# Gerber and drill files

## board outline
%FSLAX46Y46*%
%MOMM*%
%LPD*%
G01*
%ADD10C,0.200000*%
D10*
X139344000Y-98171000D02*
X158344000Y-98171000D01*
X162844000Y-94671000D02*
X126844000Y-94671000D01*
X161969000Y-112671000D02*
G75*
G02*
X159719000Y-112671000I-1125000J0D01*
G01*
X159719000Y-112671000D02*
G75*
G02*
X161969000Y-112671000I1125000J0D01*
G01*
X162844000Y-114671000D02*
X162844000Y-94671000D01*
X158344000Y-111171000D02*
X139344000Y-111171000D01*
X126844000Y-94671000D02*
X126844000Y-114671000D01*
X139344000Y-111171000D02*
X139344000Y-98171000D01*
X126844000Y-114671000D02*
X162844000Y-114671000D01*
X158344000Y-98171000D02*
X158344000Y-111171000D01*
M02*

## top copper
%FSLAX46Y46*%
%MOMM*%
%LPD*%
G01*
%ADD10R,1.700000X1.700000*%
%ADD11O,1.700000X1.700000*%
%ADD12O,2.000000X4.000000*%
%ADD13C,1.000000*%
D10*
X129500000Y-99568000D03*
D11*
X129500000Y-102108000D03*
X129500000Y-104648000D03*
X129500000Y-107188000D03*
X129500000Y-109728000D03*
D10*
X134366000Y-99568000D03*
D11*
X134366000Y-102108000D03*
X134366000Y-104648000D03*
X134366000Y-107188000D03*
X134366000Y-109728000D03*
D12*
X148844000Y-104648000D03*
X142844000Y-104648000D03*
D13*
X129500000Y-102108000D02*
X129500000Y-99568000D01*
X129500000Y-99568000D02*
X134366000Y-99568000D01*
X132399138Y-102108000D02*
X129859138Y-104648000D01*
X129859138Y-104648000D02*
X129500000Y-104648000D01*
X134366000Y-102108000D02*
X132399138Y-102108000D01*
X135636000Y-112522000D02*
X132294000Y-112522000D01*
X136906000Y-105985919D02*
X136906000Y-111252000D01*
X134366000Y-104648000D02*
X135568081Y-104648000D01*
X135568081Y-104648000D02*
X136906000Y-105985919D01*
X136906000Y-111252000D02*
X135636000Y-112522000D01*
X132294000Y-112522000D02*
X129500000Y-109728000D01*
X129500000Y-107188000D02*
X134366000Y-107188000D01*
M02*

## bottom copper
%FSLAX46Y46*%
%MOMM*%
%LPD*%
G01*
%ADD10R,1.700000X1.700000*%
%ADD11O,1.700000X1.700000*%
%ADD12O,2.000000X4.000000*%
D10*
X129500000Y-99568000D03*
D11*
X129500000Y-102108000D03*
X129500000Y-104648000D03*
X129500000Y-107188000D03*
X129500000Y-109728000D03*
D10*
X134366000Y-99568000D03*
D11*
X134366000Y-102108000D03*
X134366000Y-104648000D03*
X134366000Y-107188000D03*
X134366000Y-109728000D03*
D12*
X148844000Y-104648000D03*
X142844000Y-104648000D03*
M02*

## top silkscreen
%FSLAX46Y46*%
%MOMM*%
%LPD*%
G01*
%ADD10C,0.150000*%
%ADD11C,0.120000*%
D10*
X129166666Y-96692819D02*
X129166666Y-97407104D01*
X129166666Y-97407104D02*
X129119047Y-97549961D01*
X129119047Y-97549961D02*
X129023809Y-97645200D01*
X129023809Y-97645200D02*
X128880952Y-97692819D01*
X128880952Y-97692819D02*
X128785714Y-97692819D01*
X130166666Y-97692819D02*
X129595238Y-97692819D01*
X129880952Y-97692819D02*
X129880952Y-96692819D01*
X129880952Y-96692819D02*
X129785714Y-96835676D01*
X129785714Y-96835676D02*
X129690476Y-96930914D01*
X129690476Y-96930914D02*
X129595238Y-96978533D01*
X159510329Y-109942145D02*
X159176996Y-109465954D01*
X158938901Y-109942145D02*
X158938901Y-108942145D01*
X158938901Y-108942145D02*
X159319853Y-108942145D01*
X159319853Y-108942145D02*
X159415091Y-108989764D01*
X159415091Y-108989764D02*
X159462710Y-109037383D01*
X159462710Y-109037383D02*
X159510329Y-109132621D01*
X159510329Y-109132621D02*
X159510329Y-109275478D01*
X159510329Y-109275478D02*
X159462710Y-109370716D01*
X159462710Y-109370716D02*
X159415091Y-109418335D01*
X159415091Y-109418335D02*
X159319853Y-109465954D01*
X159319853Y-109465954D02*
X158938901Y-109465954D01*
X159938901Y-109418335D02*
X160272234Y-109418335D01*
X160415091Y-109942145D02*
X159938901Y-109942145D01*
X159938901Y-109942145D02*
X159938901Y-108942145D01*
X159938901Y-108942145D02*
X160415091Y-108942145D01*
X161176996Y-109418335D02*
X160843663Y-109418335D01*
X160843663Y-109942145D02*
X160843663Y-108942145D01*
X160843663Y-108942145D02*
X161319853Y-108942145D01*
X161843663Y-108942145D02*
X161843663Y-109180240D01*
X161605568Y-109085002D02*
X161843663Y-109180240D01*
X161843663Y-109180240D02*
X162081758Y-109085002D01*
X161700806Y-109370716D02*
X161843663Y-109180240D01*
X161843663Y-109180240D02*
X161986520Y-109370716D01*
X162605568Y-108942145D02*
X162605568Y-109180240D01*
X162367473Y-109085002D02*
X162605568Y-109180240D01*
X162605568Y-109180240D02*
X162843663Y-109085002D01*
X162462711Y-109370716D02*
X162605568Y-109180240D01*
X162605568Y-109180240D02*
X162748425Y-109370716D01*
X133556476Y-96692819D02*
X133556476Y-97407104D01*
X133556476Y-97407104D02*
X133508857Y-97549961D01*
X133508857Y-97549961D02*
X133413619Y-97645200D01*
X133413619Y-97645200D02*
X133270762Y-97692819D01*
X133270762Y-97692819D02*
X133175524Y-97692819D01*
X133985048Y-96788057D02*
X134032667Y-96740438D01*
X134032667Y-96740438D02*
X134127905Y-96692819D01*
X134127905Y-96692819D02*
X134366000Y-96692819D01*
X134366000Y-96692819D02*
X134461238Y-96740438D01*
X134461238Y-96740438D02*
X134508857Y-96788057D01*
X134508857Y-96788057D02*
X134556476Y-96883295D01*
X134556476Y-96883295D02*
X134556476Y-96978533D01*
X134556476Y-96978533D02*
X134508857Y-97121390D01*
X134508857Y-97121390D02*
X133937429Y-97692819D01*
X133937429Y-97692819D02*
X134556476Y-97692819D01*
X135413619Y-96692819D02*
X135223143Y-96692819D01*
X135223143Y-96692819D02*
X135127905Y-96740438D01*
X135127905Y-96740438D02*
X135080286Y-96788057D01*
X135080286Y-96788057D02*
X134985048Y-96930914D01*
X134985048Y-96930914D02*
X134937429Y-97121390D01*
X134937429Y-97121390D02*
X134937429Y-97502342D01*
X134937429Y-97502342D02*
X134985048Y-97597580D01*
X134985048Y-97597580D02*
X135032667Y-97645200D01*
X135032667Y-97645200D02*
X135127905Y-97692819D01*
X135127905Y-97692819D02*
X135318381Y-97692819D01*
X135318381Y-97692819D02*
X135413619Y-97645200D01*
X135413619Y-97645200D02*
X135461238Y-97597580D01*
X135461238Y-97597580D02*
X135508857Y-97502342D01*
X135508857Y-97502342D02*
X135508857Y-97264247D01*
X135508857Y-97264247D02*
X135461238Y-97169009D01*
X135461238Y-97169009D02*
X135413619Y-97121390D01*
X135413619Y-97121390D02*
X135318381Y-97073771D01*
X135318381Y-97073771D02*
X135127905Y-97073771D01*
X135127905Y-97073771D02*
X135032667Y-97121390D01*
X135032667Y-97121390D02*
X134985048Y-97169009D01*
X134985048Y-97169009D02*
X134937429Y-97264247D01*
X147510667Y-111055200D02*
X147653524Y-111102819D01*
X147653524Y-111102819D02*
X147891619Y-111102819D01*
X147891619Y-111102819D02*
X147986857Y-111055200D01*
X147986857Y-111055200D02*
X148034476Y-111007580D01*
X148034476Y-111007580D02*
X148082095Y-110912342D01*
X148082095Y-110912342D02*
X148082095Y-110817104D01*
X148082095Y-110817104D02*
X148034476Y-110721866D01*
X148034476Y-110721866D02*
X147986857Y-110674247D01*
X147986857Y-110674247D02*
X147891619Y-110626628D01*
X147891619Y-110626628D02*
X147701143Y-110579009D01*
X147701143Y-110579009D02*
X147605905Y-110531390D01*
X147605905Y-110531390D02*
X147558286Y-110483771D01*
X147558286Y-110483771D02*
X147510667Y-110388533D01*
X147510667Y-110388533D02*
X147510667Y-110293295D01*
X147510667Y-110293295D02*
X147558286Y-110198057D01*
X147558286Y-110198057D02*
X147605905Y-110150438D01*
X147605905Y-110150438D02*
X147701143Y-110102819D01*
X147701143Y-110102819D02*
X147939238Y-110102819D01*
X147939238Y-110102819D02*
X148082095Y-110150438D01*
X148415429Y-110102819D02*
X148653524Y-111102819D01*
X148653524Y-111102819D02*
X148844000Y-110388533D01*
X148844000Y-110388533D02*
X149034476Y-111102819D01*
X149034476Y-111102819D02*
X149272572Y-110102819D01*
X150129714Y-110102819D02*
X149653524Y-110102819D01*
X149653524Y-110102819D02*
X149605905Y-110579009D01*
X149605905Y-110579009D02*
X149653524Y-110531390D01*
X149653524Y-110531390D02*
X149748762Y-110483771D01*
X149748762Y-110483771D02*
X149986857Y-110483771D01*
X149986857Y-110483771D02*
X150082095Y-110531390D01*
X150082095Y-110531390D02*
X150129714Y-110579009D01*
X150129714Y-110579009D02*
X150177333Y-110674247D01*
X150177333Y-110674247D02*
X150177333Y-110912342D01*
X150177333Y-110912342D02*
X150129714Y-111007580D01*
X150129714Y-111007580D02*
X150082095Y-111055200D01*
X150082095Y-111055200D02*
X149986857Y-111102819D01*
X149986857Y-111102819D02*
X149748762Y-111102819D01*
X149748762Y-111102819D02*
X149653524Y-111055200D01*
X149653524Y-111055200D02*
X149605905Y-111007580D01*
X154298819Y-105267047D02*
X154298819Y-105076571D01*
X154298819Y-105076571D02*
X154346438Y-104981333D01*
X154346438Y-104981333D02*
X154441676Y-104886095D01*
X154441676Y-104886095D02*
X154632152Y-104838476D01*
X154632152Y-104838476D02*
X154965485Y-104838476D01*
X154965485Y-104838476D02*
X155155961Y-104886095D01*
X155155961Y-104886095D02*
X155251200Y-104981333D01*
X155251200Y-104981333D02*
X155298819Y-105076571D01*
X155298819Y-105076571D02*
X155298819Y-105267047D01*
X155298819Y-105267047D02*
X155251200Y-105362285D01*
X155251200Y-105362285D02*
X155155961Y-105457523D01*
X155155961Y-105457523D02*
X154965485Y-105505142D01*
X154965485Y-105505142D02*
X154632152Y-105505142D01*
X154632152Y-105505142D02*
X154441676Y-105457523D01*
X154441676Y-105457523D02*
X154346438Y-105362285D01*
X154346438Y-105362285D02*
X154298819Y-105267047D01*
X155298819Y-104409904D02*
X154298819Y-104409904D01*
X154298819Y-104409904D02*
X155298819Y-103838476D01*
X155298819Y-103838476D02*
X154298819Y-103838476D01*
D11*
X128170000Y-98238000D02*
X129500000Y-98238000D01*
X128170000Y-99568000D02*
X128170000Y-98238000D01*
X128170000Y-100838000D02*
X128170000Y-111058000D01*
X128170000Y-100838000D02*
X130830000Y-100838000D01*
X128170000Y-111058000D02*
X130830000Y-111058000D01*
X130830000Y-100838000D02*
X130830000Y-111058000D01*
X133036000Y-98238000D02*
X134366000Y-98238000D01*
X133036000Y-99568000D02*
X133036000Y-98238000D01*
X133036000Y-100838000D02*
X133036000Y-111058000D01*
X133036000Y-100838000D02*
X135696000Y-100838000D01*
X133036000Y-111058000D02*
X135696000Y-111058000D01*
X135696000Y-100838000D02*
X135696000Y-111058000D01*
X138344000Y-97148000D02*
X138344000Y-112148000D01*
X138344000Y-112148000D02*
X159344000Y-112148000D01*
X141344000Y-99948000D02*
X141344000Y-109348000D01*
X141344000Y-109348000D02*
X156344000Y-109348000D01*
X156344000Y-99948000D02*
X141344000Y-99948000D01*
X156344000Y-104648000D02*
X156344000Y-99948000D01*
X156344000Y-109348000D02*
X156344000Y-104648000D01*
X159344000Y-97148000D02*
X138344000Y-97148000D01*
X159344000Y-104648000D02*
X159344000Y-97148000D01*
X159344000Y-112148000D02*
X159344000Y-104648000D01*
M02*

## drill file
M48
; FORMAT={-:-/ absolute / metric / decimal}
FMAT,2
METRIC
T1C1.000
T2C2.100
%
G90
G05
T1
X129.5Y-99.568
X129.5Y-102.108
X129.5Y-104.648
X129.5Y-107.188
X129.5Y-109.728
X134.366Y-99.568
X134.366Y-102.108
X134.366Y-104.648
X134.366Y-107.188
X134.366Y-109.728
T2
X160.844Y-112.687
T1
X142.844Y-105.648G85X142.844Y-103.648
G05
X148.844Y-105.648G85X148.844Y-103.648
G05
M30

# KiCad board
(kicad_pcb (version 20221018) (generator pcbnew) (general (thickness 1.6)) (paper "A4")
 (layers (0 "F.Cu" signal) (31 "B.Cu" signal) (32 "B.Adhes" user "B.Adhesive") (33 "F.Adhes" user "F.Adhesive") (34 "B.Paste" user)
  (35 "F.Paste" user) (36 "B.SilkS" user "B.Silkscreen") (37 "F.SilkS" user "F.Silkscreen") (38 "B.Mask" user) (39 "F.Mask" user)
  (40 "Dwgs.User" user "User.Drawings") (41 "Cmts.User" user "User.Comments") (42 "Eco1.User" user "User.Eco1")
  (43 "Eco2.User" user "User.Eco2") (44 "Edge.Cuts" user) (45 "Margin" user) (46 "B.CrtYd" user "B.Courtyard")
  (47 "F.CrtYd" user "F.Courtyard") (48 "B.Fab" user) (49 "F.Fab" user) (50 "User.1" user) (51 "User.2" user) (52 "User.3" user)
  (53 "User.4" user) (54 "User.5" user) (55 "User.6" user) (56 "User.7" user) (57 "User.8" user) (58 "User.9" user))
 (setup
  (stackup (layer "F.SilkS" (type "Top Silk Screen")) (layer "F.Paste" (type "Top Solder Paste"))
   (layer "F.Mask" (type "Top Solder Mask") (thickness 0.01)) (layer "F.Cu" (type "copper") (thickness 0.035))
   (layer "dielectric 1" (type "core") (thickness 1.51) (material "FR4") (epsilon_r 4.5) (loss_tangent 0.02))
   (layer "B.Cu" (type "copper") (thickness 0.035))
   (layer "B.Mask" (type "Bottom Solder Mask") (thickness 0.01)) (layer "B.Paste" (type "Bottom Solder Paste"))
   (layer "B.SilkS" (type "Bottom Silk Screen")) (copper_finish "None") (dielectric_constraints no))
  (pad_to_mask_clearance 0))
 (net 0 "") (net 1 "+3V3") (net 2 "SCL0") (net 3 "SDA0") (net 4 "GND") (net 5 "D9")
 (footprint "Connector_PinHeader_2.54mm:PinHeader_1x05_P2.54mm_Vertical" (layer "F.Cu") (at 129.5 99.568)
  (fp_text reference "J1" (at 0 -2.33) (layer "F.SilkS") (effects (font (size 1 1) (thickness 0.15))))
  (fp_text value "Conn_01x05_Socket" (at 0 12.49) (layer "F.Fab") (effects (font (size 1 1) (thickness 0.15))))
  (fp_line (start -1.33 -1.33) (end 0 -1.33) (stroke (width 0.12) (type solid)) (layer "F.SilkS"))
  (fp_line (start -1.33 0) (end -1.33 -1.33) (stroke (width 0.12) (type solid)) (layer "F.SilkS"))
  (fp_line (start -1.33 1.27) (end -1.33 11.49) (stroke (width 0.12) (type solid)) (layer "F.SilkS"))
  (fp_line (start -1.33 1.27) (end 1.33 1.27) (stroke (width 0.12) (type solid)) (layer "F.SilkS"))
  (fp_line (start -1.33 11.49) (end 1.33 11.49) (stroke (width 0.12) (type solid)) (layer "F.SilkS"))
  (fp_line (start 1.33 1.27) (end 1.33 11.49) (stroke (width 0.12) (type solid)) (layer "F.SilkS"))
  (pad "1" thru_hole rect (at 0 0) (size 1.7 1.7) (drill 1) (layers "*.Cu" "*.Mask") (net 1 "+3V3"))
  (pad "2" thru_hole oval (at 0 2.54) (size 1.7 1.7) (drill 1) (layers "*.Cu" "*.Mask") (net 1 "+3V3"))
  (pad "3" thru_hole oval (at 0 5.08) (size 1.7 1.7) (drill 1) (layers "*.Cu" "*.Mask") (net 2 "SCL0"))
  (pad "4" thru_hole oval (at 0 7.62) (size 1.7 1.7) (drill 1) (layers "*.Cu" "*.Mask") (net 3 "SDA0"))
  (pad "5" thru_hole oval (at 0 10.16) (size 1.7 1.7) (drill 1) (layers "*.Cu" "*.Mask") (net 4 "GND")))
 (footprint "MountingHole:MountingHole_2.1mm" (layer "F.Cu") (at 160.843663 112.687326)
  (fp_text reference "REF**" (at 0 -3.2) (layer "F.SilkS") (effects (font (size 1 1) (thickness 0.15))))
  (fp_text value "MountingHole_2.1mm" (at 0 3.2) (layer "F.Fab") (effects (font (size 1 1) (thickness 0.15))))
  (pad "" np_thru_hole circle (at 0 0) (size 2.1 2.1) (drill 2.1) (layers "*.Cu" "*.Mask")))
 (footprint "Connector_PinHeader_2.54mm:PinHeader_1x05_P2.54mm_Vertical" (layer "F.Cu") (at 134.366 99.568)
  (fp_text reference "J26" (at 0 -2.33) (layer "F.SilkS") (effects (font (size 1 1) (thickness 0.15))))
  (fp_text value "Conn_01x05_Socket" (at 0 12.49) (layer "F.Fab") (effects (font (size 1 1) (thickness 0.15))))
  (fp_line (start -1.33 -1.33) (end 0 -1.33) (stroke (width 0.12) (type solid)) (layer "F.SilkS"))
  (fp_line (start -1.33 0) (end -1.33 -1.33) (stroke (width 0.12) (type solid)) (layer "F.SilkS"))
  (fp_line (start -1.33 1.27) (end -1.33 11.49) (stroke (width 0.12) (type solid)) (layer "F.SilkS"))
  (fp_line (start -1.33 1.27) (end 1.33 1.27) (stroke (width 0.12) (type solid)) (layer "F.SilkS"))
  (fp_line (start -1.33 11.49) (end 1.33 11.49) (stroke (width 0.12) (type solid)) (layer "F.SilkS"))
  (fp_line (start 1.33 1.27) (end 1.33 11.49) (stroke (width 0.12) (type solid)) (layer "F.SilkS"))
  (pad "1" thru_hole rect (at 0 0) (size 1.7 1.7) (drill 1) (layers "*.Cu" "*.Mask") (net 1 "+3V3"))
  (pad "2" thru_hole oval (at 0 2.54) (size 1.7 1.7) (drill 1) (layers "*.Cu" "*.Mask") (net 2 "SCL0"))
  (pad "3" thru_hole oval (at 0 5.08) (size 1.7 1.7) (drill 1) (layers "*.Cu" "*.Mask") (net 4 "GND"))
  (pad "4" thru_hole oval (at 0 7.62) (size 1.7 1.7) (drill 1) (layers "*.Cu" "*.Mask") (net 3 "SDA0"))
  (pad "5" thru_hole oval (at 0 10.16) (size 1.7 1.7) (drill 1) (layers "*.Cu" "*.Mask") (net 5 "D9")))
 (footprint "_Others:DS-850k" (layer "F.Cu") (at 148.844 104.648)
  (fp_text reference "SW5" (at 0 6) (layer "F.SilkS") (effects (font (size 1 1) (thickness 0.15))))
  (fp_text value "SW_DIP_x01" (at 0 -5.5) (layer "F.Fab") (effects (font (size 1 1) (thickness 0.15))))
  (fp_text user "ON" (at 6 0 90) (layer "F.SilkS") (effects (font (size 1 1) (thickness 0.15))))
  (fp_line (start -10.5 -7.5) (end -10.5 7.5) (stroke (width 0.12) (type solid)) (layer "F.SilkS"))
  (fp_line (start -10.5 7.5) (end 10.5 7.5) (stroke (width 0.12) (type solid)) (layer "F.SilkS"))
  (fp_line (start -7.5 -4.7) (end -7.5 4.7) (stroke (width 0.12) (type solid)) (layer "F.SilkS"))
  (fp_line (start -7.5 4.7) (end 7.5 4.7) (stroke (width 0.12) (type solid)) (layer "F.SilkS"))
  (fp_line (start 7.5 -4.7) (end -7.5 -4.7) (stroke (width 0.12) (type solid)) (layer "F.SilkS"))
  (fp_line (start 7.5 0) (end 7.5 -4.7) (stroke (width 0.12) (type solid)) (layer "F.SilkS"))
  (fp_line (start 7.5 4.7) (end 7.5 0) (stroke (width 0.12) (type solid)) (layer "F.SilkS"))
  (fp_line (start 10.5 -7.5) (end -10.5 -7.5) (stroke (width 0.12) (type solid)) (layer "F.SilkS"))
  (fp_line (start 10.5 0) (end 10.5 -7.5) (stroke (width 0.12) (type solid)) (layer "F.SilkS"))
  (fp_line (start 10.5 7.5) (end 10.5 0) (stroke (width 0.12) (type solid)) (layer "F.SilkS"))
  (pad "1" thru_hole oval (at 0 0 90) (size 4 2) (drill oval 3 1) (layers "*.Cu" "*.Mask") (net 1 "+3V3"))
  (pad "2" thru_hole oval (at -6 0 90) (size 4 2) (drill oval 3 1) (layers "*.Cu" "*.Mask") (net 5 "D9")))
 (gr_line (start 139.344 98.171) (end 158.344 98.171) (stroke (width 0.2) (type solid)) (layer "Edge.Cuts"))
 (gr_line (start 162.844 94.671) (end 126.844 94.671) (stroke (width 0.2) (type solid)) (layer "Edge.Cuts"))
 (gr_circle (center 160.844 112.671) (end 159.719 112.671) (stroke (width 0.2) (type solid)) (fill none) (layer "Edge.Cuts"))
 (gr_line (start 162.844 114.671) (end 162.844 94.671) (stroke (width 0.2) (type solid)) (layer "Edge.Cuts"))
 (gr_line (start 158.344 111.171) (end 139.344 111.171) (stroke (width 0.2) (type solid)) (layer "Edge.Cuts"))
 (gr_line (start 126.844 94.671) (end 126.844 114.671) (stroke (width 0.2) (type solid)) (layer "Edge.Cuts"))
 (gr_line (start 139.344 111.171) (end 139.344 98.171) (stroke (width 0.2) (type solid)) (layer "Edge.Cuts"))
 (gr_line (start 126.844 114.671) (end 162.844 114.671) (stroke (width 0.2) (type solid)) (layer "Edge.Cuts"))
 (gr_line (start 158.344 98.171) (end 158.344 111.171) (stroke (width 0.2) (type solid)) (layer "Edge.Cuts"))
 (segment (start 129.5 102.108) (end 129.5 99.568) (width 1) (layer "F.Cu") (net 1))
 (segment (start 129.5 99.568) (end 134.366 99.568) (width 1) (layer "F.Cu") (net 1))
 (segment (start 132.399138 102.108) (end 129.859138 104.648) (width 1) (layer "F.Cu") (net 2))
 (segment (start 129.859138 104.648) (end 129.5 104.648) (width 1) (layer "F.Cu") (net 2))
 (segment (start 134.366 102.108) (end 132.399138 102.108) (width 1) (layer "F.Cu") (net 2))
 (segment (start 135.636 112.522) (end 132.294 112.522) (width 1) (layer "F.Cu") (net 4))
 (segment (start 136.906 105.985919) (end 136.906 111.252) (width 1) (layer "F.Cu") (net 4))
 (segment (start 134.366 104.648) (end 135.568081 104.648) (width 1) (layer "F.Cu") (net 4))
 (segment (start 135.568081 104.648) (end 136.906 105.985919) (width 1) (layer "F.Cu") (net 4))
 (segment (start 136.906 111.252) (end 135.636 112.522) (width 1) (layer "F.Cu") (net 4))
 (segment (start 132.294 112.522) (end 129.5 109.728) (width 1) (layer "F.Cu") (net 4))
 (segment (start 129.5 107.188) (end 134.366 107.188) (width 1) (layer "F.Cu") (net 3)))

